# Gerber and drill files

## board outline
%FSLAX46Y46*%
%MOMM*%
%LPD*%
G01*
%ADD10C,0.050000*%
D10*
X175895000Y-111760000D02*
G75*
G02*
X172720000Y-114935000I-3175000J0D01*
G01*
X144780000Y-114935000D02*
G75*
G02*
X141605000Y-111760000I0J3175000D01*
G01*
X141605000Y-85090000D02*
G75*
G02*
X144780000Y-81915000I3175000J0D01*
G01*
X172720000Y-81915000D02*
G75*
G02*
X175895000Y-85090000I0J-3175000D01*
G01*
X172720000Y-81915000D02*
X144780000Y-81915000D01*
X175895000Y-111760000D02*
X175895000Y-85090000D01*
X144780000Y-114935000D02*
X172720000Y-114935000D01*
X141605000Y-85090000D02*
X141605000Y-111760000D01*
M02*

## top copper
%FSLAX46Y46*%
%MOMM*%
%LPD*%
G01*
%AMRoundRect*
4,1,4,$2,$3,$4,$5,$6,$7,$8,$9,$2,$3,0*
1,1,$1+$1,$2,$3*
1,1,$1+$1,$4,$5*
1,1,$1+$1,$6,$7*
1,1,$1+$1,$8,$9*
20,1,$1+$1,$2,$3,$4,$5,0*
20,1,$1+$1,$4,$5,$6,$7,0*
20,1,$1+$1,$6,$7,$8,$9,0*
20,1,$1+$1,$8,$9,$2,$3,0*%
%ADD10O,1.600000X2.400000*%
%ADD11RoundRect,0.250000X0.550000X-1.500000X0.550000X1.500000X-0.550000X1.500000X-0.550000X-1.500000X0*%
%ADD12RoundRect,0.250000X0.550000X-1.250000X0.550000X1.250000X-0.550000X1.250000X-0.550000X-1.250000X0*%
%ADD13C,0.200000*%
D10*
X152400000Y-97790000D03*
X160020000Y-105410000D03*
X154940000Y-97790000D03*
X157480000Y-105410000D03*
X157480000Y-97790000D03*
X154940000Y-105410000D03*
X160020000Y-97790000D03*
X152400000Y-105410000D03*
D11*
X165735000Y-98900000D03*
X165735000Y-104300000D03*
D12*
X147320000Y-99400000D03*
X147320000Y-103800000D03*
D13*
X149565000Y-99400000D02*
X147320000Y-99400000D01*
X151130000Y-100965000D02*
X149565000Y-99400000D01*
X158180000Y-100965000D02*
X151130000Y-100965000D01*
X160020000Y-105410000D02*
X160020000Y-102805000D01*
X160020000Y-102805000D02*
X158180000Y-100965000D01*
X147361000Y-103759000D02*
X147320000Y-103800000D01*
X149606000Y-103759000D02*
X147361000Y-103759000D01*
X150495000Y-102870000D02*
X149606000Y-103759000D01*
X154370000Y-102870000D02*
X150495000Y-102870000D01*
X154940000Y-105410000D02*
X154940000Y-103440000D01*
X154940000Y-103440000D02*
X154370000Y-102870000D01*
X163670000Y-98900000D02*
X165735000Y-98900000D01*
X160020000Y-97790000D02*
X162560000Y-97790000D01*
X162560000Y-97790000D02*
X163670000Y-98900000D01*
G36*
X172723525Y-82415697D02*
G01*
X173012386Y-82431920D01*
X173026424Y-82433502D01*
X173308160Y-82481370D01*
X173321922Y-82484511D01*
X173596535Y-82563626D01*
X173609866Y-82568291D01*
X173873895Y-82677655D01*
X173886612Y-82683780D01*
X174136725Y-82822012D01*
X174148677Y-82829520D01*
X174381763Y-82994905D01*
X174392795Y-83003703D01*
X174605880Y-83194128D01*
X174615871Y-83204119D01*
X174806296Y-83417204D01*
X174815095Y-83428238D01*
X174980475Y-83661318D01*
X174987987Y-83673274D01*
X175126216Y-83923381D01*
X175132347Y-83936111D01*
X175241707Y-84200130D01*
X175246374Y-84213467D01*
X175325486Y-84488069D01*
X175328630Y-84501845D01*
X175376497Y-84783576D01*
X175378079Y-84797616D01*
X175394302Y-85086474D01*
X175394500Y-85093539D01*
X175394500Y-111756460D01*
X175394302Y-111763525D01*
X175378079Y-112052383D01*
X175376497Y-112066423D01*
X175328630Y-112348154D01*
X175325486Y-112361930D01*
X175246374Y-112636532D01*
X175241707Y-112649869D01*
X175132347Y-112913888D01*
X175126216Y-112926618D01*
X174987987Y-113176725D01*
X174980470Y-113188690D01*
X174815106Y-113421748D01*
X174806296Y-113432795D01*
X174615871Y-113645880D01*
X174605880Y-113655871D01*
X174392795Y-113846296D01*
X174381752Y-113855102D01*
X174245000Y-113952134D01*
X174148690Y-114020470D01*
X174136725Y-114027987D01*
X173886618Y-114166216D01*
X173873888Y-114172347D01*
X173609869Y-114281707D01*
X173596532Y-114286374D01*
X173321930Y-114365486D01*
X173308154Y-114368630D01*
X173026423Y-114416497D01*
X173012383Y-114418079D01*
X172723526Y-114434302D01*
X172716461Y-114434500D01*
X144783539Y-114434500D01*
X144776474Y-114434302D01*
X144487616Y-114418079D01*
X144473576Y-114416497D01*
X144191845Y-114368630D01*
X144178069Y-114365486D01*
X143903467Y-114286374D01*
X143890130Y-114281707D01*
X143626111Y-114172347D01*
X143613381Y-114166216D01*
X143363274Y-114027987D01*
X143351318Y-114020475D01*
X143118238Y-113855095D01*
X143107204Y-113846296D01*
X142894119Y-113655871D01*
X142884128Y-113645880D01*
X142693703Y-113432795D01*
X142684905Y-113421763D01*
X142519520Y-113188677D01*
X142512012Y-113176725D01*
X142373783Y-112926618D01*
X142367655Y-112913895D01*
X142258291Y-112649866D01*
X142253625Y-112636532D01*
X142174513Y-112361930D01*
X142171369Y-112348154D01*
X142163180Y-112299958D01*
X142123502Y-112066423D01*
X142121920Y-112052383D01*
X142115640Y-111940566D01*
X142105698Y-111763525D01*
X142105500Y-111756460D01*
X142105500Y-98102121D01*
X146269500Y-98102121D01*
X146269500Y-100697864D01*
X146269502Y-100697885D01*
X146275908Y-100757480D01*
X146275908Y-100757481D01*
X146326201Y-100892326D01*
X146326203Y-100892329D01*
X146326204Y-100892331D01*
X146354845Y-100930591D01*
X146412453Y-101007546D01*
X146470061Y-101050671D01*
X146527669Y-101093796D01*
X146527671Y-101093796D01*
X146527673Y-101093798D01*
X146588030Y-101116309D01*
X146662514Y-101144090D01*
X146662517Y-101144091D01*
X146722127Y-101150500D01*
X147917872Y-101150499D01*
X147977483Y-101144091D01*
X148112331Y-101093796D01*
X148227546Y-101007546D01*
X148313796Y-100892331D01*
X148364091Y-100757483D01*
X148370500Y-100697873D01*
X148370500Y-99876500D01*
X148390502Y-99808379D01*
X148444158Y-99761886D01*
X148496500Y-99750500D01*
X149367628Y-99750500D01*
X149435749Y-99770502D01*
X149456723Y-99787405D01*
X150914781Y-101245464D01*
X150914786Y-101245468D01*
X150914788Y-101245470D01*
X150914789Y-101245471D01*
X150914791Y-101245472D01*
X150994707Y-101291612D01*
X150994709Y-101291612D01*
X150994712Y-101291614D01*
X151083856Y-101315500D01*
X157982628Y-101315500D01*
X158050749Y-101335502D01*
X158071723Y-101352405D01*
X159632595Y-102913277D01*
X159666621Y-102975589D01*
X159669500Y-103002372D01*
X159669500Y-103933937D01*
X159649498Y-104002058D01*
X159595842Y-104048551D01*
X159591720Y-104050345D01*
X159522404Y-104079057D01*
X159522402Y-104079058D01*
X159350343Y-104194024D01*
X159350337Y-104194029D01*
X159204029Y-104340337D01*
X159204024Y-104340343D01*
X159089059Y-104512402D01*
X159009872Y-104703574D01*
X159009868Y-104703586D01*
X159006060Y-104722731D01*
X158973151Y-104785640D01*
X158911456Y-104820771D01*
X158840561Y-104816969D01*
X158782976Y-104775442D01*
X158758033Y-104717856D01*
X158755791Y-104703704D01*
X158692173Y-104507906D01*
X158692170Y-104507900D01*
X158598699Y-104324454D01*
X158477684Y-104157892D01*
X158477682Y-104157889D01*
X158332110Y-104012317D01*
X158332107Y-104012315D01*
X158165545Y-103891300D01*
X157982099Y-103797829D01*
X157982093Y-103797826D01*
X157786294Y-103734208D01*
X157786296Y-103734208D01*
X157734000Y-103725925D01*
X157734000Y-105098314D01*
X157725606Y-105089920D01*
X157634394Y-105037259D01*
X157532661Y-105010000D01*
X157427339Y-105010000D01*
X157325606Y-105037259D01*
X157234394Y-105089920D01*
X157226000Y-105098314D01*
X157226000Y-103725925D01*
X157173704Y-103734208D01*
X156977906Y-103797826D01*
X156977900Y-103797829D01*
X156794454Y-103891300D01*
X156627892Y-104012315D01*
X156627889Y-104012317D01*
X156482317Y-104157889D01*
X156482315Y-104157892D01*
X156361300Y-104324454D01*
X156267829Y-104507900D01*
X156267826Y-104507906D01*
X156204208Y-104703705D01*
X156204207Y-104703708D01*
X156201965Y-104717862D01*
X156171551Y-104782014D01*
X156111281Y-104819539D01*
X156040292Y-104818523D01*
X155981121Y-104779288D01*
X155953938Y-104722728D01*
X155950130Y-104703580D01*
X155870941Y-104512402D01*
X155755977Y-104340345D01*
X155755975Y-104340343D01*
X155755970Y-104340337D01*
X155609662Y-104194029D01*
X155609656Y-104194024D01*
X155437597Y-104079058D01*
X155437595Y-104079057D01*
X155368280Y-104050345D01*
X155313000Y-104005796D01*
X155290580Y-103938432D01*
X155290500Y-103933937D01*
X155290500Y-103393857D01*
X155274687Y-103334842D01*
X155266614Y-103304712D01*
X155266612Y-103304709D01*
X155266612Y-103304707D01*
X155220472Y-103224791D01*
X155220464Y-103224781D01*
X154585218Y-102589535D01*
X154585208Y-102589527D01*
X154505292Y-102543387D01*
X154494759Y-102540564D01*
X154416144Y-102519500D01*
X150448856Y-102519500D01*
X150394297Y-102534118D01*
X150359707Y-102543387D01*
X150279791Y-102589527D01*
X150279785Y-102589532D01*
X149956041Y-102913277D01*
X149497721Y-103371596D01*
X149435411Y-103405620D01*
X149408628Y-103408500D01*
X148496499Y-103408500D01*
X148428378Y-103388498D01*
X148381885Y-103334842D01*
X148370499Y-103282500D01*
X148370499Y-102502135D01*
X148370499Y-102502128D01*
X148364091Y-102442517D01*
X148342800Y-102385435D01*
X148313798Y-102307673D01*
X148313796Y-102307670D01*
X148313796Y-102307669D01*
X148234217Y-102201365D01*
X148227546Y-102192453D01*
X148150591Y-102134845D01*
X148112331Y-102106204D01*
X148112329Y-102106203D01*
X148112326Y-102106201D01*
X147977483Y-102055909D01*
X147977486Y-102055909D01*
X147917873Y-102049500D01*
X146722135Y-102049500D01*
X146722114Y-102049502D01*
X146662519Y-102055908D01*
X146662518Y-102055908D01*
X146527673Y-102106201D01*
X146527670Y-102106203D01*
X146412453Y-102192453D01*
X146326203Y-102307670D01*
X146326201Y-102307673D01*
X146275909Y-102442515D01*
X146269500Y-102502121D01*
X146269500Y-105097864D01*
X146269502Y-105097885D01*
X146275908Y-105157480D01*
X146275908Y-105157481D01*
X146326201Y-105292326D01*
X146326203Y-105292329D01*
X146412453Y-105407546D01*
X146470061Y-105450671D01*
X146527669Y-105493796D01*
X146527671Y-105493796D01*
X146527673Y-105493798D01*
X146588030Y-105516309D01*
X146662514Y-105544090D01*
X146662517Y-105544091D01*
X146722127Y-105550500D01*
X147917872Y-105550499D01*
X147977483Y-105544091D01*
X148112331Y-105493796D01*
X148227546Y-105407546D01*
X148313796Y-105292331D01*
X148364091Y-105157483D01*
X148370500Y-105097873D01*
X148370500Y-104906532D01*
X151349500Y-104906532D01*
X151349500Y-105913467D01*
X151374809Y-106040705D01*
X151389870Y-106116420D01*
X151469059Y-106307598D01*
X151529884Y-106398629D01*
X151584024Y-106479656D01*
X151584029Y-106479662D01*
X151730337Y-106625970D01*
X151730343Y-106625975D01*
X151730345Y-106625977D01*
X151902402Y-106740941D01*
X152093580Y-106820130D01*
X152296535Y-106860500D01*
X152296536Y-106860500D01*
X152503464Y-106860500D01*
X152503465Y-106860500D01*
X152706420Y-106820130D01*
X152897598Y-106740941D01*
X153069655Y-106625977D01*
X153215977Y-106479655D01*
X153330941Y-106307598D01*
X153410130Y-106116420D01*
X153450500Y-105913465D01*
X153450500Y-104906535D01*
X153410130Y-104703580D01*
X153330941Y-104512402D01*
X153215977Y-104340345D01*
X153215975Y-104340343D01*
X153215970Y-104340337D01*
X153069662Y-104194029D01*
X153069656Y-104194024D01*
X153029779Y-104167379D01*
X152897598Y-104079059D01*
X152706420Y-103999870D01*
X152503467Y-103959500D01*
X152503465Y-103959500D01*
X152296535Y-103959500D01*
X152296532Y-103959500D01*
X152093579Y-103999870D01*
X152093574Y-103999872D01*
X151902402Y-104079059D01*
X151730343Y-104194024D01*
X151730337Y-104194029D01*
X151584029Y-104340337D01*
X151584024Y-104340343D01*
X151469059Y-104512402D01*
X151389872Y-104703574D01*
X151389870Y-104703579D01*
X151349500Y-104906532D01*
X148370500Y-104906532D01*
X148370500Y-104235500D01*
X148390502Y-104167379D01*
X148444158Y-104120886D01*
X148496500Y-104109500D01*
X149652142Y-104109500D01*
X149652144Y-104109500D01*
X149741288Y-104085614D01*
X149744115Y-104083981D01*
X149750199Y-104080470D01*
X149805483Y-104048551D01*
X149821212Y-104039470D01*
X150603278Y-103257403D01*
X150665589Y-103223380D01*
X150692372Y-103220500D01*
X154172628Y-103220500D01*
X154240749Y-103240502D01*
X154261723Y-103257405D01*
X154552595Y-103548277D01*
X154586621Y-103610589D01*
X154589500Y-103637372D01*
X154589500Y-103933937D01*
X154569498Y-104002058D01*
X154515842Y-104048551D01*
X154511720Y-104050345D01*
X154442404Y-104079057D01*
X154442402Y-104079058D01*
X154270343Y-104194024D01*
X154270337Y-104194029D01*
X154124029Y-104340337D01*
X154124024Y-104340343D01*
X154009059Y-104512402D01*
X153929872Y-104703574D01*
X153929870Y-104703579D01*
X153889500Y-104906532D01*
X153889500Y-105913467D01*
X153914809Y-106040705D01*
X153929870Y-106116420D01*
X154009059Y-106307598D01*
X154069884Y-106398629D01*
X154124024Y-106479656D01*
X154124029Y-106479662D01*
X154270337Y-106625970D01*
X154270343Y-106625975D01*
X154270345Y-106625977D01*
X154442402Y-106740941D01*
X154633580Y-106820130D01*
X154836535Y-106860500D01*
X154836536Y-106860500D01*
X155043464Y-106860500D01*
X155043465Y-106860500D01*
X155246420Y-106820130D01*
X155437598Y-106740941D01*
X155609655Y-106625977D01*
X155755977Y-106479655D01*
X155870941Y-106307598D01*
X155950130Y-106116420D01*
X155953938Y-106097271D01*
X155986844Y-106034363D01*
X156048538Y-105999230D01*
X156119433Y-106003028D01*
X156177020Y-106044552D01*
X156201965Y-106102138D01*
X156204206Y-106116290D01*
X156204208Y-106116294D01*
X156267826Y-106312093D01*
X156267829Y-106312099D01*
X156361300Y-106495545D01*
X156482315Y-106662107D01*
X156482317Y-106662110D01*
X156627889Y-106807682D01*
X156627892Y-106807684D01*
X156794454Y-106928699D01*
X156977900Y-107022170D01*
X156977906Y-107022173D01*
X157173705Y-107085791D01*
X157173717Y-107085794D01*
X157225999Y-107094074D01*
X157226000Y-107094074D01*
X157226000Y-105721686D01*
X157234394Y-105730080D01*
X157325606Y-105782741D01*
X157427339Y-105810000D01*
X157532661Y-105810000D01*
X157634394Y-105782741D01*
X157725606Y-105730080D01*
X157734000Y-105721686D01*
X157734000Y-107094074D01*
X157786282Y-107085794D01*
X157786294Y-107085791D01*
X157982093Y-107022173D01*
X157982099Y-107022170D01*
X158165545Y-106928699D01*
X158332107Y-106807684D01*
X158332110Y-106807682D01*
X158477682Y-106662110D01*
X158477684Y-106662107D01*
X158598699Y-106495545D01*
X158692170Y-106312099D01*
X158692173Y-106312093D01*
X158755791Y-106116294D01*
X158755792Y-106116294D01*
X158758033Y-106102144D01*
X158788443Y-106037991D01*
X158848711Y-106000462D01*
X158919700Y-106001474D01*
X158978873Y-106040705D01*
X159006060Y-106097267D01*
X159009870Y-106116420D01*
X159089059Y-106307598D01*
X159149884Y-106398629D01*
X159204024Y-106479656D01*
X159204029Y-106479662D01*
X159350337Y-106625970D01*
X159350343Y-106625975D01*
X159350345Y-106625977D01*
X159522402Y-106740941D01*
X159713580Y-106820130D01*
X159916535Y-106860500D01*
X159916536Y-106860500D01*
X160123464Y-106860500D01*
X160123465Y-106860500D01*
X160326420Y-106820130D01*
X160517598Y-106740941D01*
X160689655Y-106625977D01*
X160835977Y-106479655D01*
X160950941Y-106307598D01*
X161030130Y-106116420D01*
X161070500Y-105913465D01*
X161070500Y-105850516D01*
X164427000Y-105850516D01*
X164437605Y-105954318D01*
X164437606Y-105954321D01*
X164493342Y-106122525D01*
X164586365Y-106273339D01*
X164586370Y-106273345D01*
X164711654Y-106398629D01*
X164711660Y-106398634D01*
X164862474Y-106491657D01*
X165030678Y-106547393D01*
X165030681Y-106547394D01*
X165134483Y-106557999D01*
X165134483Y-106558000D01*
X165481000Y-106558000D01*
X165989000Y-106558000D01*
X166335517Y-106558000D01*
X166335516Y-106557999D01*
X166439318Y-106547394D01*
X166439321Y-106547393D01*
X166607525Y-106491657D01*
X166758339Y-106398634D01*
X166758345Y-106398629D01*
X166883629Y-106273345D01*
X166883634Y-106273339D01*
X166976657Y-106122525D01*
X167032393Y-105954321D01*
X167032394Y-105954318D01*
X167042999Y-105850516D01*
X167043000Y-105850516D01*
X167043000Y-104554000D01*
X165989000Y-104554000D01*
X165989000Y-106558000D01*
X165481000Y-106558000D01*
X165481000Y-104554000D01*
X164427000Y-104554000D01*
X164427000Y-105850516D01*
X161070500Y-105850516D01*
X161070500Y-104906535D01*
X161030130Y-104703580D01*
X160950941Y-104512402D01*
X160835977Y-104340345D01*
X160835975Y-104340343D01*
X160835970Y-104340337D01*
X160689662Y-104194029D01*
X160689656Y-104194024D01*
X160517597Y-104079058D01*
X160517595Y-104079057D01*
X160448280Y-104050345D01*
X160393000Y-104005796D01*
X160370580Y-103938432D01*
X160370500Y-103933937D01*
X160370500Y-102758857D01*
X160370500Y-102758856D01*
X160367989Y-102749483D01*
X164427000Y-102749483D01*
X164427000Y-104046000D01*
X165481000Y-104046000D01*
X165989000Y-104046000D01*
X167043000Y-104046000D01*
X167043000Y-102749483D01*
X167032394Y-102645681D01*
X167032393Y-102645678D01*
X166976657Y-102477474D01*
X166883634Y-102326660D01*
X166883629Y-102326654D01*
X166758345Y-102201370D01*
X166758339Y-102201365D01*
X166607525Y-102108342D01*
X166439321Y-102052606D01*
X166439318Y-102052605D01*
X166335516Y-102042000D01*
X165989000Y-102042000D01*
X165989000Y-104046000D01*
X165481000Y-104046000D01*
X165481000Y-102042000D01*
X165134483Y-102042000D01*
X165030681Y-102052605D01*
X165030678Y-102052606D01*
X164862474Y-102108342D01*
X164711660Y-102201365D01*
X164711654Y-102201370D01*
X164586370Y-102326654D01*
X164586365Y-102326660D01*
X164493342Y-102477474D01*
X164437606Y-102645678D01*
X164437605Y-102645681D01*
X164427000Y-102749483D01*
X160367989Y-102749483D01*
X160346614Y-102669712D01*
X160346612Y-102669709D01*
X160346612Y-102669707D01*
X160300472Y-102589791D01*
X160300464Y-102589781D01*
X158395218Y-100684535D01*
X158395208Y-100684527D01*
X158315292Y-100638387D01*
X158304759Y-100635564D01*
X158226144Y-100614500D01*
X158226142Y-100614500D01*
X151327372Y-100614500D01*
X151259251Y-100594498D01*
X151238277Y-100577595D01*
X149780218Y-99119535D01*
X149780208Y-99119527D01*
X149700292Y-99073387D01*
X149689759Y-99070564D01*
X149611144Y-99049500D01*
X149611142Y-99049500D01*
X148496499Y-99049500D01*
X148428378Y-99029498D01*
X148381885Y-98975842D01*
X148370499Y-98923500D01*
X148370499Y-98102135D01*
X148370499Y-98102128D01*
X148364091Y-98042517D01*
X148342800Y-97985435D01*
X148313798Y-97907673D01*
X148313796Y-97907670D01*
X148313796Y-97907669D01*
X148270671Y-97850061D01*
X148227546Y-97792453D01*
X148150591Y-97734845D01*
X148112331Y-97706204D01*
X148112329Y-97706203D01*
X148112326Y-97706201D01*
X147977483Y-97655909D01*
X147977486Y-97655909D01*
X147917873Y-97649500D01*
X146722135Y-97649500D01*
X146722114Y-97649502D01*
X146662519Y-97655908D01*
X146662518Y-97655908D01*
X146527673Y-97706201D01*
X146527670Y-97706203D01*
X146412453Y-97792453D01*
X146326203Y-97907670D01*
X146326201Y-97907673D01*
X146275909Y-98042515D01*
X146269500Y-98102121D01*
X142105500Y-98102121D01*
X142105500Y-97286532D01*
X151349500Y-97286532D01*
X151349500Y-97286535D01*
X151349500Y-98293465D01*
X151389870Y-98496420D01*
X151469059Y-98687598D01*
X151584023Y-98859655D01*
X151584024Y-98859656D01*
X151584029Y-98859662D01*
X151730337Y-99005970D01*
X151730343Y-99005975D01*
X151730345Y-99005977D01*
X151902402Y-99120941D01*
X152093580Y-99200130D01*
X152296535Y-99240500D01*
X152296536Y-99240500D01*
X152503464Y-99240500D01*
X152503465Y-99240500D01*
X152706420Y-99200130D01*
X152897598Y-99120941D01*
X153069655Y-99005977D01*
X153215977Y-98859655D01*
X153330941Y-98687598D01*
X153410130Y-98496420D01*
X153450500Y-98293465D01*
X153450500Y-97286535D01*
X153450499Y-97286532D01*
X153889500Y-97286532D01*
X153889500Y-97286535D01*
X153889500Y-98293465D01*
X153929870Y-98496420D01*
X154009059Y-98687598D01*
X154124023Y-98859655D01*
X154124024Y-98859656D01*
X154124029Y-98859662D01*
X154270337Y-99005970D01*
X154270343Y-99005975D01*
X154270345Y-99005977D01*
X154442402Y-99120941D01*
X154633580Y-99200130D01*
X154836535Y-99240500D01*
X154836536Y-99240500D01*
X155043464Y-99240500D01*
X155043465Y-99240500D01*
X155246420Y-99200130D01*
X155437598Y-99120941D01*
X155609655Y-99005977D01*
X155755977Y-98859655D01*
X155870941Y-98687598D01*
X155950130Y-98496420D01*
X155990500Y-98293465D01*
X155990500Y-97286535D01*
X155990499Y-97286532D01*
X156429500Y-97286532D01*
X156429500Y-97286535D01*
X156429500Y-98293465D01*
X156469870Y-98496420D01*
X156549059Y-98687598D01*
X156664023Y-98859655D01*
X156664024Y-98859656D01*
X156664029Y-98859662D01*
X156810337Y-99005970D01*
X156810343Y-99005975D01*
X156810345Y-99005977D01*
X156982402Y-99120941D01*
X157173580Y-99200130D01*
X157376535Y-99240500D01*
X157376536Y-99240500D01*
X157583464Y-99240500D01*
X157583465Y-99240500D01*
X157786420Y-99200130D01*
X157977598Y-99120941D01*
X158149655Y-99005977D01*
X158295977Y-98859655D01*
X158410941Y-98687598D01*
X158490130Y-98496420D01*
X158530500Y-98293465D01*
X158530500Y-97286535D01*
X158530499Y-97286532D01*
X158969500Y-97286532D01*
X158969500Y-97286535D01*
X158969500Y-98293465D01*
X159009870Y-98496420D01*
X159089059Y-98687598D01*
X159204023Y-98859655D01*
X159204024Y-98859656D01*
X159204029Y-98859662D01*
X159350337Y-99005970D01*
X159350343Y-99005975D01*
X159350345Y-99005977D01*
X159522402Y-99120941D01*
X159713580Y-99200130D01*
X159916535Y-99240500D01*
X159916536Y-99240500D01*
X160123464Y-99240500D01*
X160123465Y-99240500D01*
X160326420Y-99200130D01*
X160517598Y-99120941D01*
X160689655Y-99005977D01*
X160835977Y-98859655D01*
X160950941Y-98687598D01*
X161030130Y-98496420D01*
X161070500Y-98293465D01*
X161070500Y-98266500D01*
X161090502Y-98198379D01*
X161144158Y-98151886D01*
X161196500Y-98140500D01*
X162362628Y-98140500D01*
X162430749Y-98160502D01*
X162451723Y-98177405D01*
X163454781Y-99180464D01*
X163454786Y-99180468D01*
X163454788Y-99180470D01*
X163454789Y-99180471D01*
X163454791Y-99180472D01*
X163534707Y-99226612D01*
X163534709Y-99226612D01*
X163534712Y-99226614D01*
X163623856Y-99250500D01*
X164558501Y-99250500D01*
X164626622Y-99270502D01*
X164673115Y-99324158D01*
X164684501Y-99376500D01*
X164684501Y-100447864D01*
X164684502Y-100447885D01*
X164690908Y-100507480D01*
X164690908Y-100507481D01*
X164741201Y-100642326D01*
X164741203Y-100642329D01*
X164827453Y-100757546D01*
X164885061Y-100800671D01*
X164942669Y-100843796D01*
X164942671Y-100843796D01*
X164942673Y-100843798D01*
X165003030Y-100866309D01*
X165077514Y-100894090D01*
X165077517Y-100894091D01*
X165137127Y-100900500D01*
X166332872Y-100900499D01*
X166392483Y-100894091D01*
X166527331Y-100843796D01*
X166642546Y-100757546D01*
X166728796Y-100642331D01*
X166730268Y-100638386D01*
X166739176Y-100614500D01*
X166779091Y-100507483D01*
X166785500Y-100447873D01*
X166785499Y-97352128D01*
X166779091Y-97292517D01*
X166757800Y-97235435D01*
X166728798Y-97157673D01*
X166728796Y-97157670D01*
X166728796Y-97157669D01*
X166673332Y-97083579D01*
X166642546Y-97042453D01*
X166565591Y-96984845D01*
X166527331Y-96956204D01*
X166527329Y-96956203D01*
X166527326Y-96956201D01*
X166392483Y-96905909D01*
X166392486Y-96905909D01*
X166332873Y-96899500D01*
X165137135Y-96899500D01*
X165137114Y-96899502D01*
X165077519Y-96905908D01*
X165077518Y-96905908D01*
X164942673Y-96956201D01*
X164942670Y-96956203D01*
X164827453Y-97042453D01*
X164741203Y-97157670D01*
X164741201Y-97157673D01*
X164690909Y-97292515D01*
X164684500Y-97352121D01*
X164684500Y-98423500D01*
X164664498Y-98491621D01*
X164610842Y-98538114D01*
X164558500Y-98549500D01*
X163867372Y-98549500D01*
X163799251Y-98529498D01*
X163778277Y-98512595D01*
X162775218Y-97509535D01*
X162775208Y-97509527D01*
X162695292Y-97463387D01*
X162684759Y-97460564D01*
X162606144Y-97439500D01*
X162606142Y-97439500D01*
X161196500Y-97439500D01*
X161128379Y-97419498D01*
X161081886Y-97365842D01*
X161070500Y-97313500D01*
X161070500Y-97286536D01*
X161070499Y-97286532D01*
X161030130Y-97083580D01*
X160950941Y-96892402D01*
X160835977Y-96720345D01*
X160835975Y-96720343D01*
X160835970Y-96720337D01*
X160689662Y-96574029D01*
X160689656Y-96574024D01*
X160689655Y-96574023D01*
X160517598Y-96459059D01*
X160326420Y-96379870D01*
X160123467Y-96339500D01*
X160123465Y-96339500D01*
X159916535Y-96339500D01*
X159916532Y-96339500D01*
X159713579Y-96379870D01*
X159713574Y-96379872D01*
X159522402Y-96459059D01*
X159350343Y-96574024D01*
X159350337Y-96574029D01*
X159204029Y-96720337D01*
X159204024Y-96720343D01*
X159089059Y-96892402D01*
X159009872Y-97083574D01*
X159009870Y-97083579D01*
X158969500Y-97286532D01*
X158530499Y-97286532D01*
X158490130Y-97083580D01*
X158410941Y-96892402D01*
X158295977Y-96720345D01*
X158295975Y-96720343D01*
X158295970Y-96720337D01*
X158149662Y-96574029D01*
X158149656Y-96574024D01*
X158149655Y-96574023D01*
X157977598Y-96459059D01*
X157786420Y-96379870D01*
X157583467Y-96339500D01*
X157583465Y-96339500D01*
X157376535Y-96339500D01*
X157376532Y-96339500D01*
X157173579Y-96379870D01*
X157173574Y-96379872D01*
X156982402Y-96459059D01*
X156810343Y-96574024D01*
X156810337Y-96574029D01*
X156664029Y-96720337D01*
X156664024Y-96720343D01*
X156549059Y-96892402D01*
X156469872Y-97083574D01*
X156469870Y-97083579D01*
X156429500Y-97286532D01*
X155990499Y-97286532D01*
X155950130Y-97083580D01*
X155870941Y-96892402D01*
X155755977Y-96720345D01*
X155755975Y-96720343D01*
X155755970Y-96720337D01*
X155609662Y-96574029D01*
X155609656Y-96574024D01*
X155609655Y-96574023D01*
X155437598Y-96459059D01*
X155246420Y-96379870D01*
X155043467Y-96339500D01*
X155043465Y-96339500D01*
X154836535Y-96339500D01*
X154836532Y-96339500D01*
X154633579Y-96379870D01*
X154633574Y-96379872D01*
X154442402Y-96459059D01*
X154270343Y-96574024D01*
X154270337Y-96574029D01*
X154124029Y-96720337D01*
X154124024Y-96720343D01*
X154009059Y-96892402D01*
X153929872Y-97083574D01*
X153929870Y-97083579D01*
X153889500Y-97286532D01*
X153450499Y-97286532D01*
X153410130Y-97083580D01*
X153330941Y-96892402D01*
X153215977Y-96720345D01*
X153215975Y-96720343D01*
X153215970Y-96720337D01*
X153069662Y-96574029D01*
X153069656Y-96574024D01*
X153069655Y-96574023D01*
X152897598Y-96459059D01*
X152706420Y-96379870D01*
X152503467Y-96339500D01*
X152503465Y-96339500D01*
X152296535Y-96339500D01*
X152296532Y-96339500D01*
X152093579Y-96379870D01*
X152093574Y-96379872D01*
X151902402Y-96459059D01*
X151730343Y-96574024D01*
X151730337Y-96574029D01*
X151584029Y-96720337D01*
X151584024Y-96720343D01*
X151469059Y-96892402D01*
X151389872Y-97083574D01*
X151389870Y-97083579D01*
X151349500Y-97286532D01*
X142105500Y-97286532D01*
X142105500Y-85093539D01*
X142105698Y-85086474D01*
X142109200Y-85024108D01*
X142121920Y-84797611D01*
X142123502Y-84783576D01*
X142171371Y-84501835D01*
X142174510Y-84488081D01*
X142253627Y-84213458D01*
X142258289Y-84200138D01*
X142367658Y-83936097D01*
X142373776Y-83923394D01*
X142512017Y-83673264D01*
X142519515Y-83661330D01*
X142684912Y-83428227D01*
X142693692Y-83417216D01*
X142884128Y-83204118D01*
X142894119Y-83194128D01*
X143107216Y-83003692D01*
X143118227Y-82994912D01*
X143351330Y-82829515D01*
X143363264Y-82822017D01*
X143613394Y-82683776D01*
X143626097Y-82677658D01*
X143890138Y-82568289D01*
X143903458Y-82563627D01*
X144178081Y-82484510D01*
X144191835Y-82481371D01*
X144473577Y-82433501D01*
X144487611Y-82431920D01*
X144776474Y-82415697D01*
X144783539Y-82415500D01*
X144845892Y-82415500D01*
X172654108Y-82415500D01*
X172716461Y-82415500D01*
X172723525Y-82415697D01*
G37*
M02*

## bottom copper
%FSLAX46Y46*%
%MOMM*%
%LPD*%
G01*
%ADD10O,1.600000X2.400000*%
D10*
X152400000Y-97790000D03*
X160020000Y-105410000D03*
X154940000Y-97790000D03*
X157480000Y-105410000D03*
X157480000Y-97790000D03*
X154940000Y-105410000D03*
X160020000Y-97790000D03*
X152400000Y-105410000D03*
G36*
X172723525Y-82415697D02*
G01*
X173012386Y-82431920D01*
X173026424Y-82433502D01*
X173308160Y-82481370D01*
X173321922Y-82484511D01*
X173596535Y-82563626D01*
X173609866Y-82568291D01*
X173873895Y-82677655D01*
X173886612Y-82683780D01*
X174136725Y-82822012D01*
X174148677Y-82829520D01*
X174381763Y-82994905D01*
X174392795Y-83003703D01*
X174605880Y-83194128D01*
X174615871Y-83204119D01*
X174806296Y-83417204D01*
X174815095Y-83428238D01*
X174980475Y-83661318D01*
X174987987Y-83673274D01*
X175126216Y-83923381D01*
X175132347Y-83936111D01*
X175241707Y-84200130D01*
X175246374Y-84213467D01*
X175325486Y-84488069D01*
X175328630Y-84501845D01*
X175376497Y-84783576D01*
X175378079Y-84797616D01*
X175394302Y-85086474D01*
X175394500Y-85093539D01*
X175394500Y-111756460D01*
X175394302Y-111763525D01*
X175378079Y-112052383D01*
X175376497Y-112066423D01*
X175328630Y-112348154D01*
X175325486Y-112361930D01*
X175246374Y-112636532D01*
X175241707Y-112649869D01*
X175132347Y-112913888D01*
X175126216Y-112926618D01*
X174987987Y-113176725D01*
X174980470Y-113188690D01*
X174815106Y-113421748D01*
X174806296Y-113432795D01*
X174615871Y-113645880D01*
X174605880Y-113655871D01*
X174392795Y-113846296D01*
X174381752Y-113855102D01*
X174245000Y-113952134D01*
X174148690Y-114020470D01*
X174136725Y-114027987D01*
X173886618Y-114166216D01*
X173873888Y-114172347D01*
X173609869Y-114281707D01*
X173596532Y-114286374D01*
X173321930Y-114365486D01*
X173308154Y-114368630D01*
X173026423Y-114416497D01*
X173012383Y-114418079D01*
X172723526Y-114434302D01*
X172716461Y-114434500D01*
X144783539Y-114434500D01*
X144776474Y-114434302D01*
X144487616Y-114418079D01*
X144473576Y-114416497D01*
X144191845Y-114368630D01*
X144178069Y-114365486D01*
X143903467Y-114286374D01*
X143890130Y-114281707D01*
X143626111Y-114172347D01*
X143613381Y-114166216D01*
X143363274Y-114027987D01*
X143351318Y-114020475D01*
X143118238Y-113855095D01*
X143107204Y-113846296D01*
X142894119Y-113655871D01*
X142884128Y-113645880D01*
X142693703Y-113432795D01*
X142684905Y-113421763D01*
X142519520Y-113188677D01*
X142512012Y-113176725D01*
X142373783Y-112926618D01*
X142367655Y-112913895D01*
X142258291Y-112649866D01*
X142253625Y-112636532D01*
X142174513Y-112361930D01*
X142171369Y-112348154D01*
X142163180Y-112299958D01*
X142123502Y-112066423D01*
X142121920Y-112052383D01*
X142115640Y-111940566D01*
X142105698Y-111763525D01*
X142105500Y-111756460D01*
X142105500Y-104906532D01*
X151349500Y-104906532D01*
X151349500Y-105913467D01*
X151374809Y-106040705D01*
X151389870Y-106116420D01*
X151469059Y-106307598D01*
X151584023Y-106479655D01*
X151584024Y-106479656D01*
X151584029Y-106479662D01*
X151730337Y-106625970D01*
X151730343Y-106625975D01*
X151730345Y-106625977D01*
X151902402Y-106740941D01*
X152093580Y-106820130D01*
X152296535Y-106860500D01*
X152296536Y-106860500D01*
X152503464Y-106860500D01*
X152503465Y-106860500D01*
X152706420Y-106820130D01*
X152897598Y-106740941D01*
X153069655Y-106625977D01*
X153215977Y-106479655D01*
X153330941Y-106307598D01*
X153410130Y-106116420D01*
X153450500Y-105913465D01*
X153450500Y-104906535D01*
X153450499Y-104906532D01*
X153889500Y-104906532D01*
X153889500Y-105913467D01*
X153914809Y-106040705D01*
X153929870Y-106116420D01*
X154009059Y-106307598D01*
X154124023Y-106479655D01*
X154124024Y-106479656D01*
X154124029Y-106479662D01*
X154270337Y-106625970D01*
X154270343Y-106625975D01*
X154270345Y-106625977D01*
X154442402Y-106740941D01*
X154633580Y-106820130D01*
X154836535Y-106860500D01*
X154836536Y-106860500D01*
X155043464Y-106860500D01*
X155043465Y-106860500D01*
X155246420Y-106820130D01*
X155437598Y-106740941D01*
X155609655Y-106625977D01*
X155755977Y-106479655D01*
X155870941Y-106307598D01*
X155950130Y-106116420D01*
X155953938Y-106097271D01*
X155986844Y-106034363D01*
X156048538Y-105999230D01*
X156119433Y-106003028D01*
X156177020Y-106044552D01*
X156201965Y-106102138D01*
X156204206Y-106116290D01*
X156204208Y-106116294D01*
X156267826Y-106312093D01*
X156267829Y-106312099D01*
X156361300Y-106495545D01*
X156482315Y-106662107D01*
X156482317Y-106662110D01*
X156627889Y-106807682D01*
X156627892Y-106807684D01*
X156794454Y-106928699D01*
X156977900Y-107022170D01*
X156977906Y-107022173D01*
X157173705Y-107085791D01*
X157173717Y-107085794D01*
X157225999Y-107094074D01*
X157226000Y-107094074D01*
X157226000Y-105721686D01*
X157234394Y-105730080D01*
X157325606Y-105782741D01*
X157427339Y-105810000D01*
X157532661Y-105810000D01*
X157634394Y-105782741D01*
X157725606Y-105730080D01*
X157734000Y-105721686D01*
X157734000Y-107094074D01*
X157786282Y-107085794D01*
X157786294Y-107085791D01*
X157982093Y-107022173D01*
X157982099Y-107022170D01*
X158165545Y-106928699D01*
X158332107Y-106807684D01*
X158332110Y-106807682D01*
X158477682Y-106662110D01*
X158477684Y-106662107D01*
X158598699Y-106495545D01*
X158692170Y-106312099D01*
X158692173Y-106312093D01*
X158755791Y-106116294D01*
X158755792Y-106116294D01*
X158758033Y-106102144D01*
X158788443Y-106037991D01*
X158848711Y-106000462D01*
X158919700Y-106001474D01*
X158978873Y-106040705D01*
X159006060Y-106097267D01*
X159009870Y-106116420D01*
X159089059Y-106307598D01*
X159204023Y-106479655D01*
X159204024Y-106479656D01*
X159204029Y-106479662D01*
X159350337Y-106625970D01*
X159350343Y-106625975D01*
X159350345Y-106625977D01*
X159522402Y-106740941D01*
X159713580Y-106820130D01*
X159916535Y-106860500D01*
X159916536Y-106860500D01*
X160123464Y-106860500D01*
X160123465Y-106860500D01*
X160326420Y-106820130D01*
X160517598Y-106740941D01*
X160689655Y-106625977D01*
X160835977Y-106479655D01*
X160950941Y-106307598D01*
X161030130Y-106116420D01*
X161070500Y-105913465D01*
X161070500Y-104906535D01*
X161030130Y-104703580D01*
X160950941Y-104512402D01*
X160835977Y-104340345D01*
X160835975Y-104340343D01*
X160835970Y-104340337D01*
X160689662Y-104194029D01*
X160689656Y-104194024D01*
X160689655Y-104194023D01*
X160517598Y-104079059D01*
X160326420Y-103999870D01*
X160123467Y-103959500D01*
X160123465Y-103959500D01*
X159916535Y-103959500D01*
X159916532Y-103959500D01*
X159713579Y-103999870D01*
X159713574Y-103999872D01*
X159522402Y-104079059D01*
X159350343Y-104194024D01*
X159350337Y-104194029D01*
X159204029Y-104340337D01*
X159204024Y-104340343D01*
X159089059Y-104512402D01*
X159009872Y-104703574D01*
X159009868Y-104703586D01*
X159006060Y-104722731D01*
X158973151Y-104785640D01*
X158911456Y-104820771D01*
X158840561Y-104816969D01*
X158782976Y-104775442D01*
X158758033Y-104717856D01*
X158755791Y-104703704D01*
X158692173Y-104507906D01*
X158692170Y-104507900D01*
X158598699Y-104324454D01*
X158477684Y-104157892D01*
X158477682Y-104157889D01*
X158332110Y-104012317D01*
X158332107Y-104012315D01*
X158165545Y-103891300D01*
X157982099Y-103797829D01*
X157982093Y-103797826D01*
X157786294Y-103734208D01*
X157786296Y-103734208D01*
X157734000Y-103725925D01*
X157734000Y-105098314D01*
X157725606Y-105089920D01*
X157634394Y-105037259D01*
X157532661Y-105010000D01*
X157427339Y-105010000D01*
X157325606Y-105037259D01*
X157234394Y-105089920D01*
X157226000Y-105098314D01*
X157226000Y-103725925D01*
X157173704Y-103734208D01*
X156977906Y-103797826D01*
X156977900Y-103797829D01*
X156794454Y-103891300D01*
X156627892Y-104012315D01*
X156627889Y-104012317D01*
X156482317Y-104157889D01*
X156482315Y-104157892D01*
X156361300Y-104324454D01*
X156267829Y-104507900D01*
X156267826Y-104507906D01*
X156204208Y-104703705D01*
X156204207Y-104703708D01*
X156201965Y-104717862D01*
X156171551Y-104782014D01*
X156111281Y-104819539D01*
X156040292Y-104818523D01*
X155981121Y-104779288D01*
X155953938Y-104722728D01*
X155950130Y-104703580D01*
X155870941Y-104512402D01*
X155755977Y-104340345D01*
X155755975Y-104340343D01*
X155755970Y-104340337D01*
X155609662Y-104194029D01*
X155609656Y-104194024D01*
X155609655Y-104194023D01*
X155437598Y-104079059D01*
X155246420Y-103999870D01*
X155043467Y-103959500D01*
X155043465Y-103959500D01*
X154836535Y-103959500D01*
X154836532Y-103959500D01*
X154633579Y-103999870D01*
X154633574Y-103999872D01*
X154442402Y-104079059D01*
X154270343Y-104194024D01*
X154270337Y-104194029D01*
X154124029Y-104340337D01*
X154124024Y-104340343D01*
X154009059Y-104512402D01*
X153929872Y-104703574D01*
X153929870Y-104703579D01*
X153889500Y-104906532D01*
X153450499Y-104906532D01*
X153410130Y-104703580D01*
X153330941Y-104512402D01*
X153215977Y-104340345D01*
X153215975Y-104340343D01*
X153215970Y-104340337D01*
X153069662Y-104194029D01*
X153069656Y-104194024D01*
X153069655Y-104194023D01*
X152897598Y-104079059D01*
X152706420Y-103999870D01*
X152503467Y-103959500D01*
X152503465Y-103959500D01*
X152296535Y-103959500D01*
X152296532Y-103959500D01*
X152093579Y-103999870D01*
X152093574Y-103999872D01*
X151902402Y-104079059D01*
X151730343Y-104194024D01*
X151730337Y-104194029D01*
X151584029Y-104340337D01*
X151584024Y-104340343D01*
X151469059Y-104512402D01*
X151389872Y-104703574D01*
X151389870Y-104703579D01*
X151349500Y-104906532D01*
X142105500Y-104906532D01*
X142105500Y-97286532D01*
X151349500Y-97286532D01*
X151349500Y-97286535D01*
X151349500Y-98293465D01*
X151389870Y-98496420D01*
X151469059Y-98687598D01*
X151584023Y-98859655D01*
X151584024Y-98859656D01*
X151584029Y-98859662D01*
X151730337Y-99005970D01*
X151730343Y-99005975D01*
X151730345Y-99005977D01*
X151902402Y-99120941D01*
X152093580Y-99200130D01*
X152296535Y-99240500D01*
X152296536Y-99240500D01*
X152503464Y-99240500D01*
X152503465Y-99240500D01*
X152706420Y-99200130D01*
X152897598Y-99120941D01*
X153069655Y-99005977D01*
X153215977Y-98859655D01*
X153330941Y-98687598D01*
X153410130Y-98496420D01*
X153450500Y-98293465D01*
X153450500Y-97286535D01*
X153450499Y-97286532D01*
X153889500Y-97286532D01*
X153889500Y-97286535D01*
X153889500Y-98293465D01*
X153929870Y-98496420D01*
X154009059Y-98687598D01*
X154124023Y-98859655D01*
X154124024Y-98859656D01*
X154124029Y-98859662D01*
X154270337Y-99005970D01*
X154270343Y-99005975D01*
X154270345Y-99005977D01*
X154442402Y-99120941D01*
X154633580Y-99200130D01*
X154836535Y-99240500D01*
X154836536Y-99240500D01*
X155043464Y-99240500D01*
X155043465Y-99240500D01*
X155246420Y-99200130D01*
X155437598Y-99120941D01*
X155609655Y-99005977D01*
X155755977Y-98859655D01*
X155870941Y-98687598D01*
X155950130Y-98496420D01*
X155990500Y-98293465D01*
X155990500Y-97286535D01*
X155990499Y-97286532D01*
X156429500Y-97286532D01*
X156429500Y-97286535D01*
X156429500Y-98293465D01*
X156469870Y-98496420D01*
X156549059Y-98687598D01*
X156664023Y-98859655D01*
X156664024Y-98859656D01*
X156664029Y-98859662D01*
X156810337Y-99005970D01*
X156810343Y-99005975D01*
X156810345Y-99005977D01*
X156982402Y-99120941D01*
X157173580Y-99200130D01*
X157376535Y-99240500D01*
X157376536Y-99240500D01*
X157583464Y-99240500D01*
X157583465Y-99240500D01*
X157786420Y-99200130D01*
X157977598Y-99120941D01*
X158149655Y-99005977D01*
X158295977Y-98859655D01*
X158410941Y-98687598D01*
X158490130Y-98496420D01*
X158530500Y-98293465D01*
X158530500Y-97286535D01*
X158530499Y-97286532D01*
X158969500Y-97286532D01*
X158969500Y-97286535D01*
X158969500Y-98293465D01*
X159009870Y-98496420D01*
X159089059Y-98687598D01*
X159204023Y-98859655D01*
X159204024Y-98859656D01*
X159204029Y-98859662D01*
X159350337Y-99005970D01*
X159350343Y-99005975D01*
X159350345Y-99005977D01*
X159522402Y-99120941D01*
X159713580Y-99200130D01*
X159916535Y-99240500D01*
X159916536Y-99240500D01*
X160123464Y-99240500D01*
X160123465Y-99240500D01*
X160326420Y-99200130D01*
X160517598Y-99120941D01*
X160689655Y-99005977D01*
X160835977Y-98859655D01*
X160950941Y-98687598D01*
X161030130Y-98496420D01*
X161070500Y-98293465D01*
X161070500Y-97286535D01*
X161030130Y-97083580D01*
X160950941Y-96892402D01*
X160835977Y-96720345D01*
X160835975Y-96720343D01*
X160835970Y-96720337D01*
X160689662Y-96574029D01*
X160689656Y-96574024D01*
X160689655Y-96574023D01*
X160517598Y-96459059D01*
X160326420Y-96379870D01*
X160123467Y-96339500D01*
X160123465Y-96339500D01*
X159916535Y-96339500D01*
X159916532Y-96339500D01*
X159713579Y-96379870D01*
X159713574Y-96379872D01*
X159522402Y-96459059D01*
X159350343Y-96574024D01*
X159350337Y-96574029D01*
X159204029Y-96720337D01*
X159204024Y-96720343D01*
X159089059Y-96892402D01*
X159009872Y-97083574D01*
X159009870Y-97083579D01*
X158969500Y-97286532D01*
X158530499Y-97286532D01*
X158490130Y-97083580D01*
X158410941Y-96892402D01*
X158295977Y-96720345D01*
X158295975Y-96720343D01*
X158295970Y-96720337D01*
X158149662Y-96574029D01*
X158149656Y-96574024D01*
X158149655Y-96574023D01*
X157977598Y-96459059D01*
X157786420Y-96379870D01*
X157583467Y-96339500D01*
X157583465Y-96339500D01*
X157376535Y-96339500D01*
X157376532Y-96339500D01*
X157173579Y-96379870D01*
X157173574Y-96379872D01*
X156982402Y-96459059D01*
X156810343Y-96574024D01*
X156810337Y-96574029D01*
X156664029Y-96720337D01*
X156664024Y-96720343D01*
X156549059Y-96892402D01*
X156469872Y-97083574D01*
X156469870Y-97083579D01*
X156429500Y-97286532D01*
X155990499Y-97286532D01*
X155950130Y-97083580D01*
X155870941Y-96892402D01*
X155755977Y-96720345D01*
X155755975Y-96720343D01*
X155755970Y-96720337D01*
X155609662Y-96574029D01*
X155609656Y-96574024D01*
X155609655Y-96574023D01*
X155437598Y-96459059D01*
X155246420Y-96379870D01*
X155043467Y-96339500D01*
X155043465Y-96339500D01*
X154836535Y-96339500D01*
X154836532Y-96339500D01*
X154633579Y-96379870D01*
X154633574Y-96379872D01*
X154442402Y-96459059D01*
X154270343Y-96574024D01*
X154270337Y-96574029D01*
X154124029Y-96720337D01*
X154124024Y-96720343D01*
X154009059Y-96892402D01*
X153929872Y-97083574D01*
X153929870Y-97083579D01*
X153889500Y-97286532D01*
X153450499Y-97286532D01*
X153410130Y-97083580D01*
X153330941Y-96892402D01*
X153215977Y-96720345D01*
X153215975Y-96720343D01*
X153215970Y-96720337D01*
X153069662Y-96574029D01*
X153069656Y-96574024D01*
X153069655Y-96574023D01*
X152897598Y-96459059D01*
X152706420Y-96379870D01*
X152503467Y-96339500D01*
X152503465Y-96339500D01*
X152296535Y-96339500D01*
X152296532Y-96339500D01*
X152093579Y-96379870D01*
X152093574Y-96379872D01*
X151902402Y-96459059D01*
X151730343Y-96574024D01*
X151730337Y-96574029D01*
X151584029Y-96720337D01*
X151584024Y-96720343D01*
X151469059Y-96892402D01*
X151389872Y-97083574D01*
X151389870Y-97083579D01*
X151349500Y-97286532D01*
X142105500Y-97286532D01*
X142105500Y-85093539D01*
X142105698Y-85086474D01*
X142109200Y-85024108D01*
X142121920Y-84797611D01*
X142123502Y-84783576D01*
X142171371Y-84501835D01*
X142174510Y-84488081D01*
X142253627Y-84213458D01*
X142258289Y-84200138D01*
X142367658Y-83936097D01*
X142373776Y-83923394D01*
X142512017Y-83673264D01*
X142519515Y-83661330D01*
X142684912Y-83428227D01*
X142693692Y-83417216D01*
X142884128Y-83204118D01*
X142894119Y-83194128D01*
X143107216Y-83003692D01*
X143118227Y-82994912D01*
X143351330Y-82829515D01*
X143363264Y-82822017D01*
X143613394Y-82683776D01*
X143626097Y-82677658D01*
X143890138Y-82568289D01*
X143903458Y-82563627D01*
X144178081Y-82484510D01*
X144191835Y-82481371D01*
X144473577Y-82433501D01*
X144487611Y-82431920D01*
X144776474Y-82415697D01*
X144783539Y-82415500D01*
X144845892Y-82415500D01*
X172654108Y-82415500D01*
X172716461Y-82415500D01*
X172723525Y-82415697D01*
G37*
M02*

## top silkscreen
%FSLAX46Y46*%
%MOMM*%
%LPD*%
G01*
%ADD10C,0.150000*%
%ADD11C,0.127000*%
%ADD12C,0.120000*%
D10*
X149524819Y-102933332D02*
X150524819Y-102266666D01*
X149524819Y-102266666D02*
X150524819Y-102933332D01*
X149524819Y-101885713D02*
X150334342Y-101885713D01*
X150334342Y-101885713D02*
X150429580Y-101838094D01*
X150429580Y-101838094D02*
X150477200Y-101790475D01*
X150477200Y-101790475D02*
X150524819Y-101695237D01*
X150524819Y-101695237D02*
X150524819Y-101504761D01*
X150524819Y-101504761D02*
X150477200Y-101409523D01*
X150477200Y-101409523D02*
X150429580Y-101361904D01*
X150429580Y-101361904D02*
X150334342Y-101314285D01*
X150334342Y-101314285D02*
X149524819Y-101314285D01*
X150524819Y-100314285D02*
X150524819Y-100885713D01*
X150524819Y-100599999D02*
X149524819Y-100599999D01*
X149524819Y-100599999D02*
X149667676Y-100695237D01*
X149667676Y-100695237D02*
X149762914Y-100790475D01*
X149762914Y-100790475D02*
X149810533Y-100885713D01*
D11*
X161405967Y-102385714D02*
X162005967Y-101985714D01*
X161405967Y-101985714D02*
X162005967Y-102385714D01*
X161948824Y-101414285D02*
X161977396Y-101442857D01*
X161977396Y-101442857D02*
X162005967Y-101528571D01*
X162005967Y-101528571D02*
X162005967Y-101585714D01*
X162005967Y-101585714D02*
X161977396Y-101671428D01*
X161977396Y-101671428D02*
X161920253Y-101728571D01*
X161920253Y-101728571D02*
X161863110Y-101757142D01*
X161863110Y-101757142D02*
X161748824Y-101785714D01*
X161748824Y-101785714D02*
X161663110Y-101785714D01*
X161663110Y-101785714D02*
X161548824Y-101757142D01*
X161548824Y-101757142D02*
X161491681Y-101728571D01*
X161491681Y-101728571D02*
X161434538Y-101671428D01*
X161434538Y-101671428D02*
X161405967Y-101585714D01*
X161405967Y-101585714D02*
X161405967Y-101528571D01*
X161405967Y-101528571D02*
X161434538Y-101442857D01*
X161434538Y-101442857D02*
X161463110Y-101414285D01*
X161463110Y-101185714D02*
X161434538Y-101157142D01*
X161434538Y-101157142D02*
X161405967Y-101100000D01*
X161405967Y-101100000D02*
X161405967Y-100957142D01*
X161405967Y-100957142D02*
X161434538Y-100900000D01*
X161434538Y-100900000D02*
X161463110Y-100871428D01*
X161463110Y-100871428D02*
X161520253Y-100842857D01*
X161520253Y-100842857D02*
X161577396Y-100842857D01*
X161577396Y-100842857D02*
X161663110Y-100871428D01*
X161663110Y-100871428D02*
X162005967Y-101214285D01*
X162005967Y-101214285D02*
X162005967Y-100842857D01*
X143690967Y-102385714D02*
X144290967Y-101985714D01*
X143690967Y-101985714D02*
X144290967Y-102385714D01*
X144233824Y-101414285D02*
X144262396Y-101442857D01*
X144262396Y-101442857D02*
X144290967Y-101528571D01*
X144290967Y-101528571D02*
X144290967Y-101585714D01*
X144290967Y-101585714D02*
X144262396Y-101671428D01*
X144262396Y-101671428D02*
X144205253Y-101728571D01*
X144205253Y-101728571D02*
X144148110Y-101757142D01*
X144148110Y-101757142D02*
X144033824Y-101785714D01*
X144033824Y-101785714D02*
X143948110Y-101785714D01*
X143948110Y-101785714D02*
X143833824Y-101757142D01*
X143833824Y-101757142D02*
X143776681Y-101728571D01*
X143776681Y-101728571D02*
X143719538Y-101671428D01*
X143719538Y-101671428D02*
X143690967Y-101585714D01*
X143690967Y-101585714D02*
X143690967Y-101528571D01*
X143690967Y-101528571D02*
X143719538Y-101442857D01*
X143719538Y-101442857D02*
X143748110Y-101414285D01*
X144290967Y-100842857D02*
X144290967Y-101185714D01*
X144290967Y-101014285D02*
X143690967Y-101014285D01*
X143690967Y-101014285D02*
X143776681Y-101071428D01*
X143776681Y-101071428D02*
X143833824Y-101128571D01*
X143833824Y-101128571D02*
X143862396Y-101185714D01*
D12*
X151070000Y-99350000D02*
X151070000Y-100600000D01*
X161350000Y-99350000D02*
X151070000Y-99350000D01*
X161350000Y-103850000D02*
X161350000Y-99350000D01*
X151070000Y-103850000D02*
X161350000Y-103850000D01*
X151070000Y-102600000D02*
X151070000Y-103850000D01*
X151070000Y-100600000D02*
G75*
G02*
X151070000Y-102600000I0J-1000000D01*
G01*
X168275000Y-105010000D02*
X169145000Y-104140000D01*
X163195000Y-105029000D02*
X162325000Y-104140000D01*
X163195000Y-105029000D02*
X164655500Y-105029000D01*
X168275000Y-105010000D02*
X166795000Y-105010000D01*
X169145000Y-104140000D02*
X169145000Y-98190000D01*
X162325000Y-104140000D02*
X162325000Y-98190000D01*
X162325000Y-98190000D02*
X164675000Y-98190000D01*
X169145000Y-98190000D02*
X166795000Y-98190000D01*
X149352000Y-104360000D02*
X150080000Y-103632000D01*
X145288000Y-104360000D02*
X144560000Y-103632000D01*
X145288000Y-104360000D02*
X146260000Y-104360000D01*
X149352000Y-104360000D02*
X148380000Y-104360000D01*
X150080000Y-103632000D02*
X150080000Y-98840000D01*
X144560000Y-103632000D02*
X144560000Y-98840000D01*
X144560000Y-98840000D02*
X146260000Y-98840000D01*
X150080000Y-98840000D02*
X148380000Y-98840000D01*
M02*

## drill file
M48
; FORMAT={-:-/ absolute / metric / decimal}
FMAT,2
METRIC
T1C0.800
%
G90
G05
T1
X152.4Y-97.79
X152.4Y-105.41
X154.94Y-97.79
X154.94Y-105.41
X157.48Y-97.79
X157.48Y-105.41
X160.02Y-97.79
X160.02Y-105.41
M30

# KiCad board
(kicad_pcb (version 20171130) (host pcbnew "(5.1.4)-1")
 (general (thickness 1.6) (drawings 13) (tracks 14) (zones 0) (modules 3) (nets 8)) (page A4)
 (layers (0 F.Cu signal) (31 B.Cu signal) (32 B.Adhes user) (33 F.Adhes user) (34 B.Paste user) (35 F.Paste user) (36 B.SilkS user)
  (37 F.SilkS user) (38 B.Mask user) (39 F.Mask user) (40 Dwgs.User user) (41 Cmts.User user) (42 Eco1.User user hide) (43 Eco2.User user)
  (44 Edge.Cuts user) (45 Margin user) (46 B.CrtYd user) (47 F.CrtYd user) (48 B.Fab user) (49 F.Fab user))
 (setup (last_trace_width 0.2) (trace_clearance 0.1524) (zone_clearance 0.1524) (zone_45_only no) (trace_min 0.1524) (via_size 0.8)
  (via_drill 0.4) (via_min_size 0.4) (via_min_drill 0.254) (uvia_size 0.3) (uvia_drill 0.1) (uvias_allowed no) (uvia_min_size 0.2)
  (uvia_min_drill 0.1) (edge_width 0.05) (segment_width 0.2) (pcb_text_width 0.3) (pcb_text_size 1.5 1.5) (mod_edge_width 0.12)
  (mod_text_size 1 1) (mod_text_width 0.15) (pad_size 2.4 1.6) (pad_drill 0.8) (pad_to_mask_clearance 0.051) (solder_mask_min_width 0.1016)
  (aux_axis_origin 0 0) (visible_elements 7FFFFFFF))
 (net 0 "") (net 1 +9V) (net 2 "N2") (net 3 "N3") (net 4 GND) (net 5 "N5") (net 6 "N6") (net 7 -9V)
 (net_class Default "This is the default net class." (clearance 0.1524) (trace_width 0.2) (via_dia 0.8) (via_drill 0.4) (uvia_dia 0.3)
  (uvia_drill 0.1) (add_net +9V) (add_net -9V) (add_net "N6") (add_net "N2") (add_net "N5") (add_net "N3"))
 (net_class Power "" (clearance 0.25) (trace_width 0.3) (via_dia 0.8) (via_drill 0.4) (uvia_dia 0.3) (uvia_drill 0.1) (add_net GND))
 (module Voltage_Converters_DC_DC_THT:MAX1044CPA (layer F.Cu) (at 156.21 101.6 90)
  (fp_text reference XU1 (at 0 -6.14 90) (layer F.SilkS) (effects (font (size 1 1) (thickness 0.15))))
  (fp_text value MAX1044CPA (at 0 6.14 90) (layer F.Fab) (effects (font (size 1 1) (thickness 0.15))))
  (fp_line (start 2.25 -5.14) (end 1 -5.14) (layer F.SilkS) (width 0.12))
  (fp_line (start 2.25 5.14) (end 2.25 -5.14) (layer F.SilkS) (width 0.12))
  (fp_line (start -2.25 5.14) (end 2.25 5.14) (layer F.SilkS) (width 0.12))
  (fp_line (start -2.25 -5.14) (end -2.25 5.14) (layer F.SilkS) (width 0.12))
  (fp_line (start -1 -5.14) (end -2.25 -5.14) (layer F.SilkS) (width 0.12))
  (fp_arc (start 0 -5.14) (end -1 -5.14) (angle -180) (layer F.SilkS) (width 0.12))
  (pad 8 thru_hole oval (at 3.81 -3.81 90) (size 2.4 1.6) (drill 0.8) (layers *.Cu *.Mask) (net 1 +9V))
  (pad 4 thru_hole oval (at -3.81 3.81 90) (size 2.4 1.6) (drill 0.8) (layers *.Cu *.Mask) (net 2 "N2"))
  (pad 7 thru_hole oval (at 3.81 -1.27 90) (size 2.4 1.6) (drill 0.8) (layers *.Cu *.Mask) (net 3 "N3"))
  (pad 3 thru_hole oval (at -3.81 1.27 90) (size 2.4 1.6) (drill 0.8) (layers *.Cu *.Mask) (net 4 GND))
  (pad 6 thru_hole oval (at 3.81 1.27 90) (size 2.4 1.6) (drill 0.8) (layers *.Cu *.Mask) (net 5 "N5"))
  (pad 2 thru_hole oval (at -3.81 -1.27 90) (size 2.4 1.6) (drill 0.8) (layers *.Cu *.Mask) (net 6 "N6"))
  (pad 5 thru_hole oval (at 3.81 3.81 90) (size 2.4 1.6) (drill 0.8) (layers *.Cu *.Mask) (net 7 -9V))
  (pad 1 thru_hole oval (at -3.81 -3.81 90) (size 2.4 1.6) (drill 0.8) (layers *.Cu *.Mask) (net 1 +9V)))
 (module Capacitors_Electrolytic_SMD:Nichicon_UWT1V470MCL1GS (layer F.Cu) (at 165.735 101.6 90)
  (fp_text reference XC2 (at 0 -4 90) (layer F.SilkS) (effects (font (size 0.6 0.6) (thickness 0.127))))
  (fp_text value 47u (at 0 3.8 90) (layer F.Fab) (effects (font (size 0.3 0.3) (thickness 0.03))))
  (fp_line (start -3.41 2.54) (end -2.54 3.41) (layer F.SilkS) (width 0.12))
  (fp_line (start -3.429 -2.54) (end -2.54 -3.41) (layer F.SilkS) (width 0.12))
  (fp_line (start -3.429 -2.54) (end -3.429 -1.0795) (layer F.SilkS) (width 0.12))
  (fp_line (start -3.41 2.54) (end -3.41 1.06) (layer F.SilkS) (width 0.12))
  (fp_line (start -2.54 3.41) (end 3.41 3.41) (layer F.SilkS) (width 0.12))
  (fp_line (start -2.54 -3.41) (end 3.41 -3.41) (layer F.SilkS) (width 0.12))
  (fp_line (start 3.41 -3.41) (end 3.41 -1.06) (layer F.SilkS) (width 0.12))
  (fp_line (start 3.41 3.41) (end 3.41 1.06) (layer F.SilkS) (width 0.12))
  (pad 2 smd roundrect (at 2.7 0 90) (size 3.5 1.6) (layers F.Cu F.Paste F.Mask) (roundrect_rratio 0.15625) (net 7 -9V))
  (pad 1 smd roundrect (at -2.7 0 90) (size 3.5 1.6) (layers F.Cu F.Paste F.Mask) (roundrect_rratio 0.15625) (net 4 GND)))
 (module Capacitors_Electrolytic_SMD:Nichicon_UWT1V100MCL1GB (layer F.Cu) (at 147.32 101.6 90)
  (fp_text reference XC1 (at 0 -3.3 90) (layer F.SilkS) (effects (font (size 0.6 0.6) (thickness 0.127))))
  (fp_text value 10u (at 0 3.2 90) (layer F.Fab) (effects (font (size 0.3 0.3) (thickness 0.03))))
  (fp_line (start -2.76 2.032) (end -2.032 2.76) (layer F.SilkS) (width 0.12))
  (fp_line (start -2.76 -2.032) (end -2.032 -2.76) (layer F.SilkS) (width 0.12))
  (fp_line (start -2.76 -2.032) (end -2.76 -1.06) (layer F.SilkS) (width 0.12))
  (fp_line (start -2.76 2.032) (end -2.76 1.06) (layer F.SilkS) (width 0.12))
  (fp_line (start -2.032 2.76) (end 2.76 2.76) (layer F.SilkS) (width 0.12))
  (fp_line (start -2.032 -2.76) (end 2.76 -2.76) (layer F.SilkS) (width 0.12))
  (fp_line (start 2.76 -2.76) (end 2.76 -1.06) (layer F.SilkS) (width 0.12))
  (fp_line (start 2.76 2.76) (end 2.76 1.06) (layer F.SilkS) (width 0.12))
  (pad 2 smd roundrect (at 2.2 0 90) (size 3 1.6) (layers F.Cu F.Paste F.Mask) (roundrect_rratio 0.15625) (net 2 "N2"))
  (pad 1 smd roundrect (at -2.2 0 90) (size 3 1.6) (layers F.Cu F.Paste F.Mask) (roundrect_rratio 0.15625) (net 6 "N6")))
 (gr_arc (start 172.72 111.76) (end 172.72 114.935) (angle -90) (layer Edge.Cuts) (width 0.05))
 (gr_arc (start 144.78 111.76) (end 141.605 111.76) (angle -90) (layer Edge.Cuts) (width 0.05))
 (gr_arc (start 144.78 85.09) (end 144.78 81.915) (angle -90) (layer Edge.Cuts) (width 0.05))
 (gr_arc (start 172.72 85.09) (end 175.895 85.09) (angle -90) (layer Edge.Cuts) (width 0.05))
 (gr_line (start 172.72 81.915) (end 144.78 81.915) (layer Edge.Cuts) (width 0.05))
 (gr_line (start 175.895 111.76) (end 175.895 85.09) (layer Edge.Cuts) (width 0.05))
 (gr_line (start 144.78 114.935) (end 172.72 114.935) (layer Edge.Cuts) (width 0.05))
 (gr_line (start 141.605 85.09) (end 141.605 111.76) (layer Edge.Cuts) (width 0.05))
 (segment (start 149.565 99.4) (end 147.32 99.4) (width 0.2) (layer F.Cu) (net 2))
 (segment (start 151.13 100.965) (end 149.565 99.4) (width 0.2) (layer F.Cu) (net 2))
 (segment (start 158.18 100.965) (end 151.13 100.965) (width 0.2) (layer F.Cu) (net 2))
 (segment (start 160.02 105.41) (end 160.02 102.805) (width 0.2) (layer F.Cu) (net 2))
 (segment (start 160.02 102.805) (end 158.18 100.965) (width 0.2) (layer F.Cu) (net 2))
 (segment (start 147.361 103.759) (end 147.32 103.8) (width 0.2) (layer F.Cu) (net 6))
 (segment (start 149.606 103.759) (end 147.361 103.759) (width 0.2) (layer F.Cu) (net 6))
 (segment (start 150.495 102.87) (end 149.606 103.759) (width 0.2) (layer F.Cu) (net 6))
 (segment (start 154.37 102.87) (end 150.495 102.87) (width 0.2) (layer F.Cu) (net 6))
 (segment (start 154.94 105.41) (end 154.94 103.44) (width 0.2) (layer F.Cu) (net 6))
 (segment (start 154.94 103.44) (end 154.37 102.87) (width 0.2) (layer F.Cu) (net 6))
 (segment (start 163.67 98.9) (end 165.735 98.9) (width 0.2) (layer F.Cu) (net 7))
 (segment (start 160.02 97.79) (end 162.56 97.79) (width 0.2) (layer F.Cu) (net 7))
 (segment (start 162.56 97.79) (end 163.67 98.9) (width 0.2) (layer F.Cu) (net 7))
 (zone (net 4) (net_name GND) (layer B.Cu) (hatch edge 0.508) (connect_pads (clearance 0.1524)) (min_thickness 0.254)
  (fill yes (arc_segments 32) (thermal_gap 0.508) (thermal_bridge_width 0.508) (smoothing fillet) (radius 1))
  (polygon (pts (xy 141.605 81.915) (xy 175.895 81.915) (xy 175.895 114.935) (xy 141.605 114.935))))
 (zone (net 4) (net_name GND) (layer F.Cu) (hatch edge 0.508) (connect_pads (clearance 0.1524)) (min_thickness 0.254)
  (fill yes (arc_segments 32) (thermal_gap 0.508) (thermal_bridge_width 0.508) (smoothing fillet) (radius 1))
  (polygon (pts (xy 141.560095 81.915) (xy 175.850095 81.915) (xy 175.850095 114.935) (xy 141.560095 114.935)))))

